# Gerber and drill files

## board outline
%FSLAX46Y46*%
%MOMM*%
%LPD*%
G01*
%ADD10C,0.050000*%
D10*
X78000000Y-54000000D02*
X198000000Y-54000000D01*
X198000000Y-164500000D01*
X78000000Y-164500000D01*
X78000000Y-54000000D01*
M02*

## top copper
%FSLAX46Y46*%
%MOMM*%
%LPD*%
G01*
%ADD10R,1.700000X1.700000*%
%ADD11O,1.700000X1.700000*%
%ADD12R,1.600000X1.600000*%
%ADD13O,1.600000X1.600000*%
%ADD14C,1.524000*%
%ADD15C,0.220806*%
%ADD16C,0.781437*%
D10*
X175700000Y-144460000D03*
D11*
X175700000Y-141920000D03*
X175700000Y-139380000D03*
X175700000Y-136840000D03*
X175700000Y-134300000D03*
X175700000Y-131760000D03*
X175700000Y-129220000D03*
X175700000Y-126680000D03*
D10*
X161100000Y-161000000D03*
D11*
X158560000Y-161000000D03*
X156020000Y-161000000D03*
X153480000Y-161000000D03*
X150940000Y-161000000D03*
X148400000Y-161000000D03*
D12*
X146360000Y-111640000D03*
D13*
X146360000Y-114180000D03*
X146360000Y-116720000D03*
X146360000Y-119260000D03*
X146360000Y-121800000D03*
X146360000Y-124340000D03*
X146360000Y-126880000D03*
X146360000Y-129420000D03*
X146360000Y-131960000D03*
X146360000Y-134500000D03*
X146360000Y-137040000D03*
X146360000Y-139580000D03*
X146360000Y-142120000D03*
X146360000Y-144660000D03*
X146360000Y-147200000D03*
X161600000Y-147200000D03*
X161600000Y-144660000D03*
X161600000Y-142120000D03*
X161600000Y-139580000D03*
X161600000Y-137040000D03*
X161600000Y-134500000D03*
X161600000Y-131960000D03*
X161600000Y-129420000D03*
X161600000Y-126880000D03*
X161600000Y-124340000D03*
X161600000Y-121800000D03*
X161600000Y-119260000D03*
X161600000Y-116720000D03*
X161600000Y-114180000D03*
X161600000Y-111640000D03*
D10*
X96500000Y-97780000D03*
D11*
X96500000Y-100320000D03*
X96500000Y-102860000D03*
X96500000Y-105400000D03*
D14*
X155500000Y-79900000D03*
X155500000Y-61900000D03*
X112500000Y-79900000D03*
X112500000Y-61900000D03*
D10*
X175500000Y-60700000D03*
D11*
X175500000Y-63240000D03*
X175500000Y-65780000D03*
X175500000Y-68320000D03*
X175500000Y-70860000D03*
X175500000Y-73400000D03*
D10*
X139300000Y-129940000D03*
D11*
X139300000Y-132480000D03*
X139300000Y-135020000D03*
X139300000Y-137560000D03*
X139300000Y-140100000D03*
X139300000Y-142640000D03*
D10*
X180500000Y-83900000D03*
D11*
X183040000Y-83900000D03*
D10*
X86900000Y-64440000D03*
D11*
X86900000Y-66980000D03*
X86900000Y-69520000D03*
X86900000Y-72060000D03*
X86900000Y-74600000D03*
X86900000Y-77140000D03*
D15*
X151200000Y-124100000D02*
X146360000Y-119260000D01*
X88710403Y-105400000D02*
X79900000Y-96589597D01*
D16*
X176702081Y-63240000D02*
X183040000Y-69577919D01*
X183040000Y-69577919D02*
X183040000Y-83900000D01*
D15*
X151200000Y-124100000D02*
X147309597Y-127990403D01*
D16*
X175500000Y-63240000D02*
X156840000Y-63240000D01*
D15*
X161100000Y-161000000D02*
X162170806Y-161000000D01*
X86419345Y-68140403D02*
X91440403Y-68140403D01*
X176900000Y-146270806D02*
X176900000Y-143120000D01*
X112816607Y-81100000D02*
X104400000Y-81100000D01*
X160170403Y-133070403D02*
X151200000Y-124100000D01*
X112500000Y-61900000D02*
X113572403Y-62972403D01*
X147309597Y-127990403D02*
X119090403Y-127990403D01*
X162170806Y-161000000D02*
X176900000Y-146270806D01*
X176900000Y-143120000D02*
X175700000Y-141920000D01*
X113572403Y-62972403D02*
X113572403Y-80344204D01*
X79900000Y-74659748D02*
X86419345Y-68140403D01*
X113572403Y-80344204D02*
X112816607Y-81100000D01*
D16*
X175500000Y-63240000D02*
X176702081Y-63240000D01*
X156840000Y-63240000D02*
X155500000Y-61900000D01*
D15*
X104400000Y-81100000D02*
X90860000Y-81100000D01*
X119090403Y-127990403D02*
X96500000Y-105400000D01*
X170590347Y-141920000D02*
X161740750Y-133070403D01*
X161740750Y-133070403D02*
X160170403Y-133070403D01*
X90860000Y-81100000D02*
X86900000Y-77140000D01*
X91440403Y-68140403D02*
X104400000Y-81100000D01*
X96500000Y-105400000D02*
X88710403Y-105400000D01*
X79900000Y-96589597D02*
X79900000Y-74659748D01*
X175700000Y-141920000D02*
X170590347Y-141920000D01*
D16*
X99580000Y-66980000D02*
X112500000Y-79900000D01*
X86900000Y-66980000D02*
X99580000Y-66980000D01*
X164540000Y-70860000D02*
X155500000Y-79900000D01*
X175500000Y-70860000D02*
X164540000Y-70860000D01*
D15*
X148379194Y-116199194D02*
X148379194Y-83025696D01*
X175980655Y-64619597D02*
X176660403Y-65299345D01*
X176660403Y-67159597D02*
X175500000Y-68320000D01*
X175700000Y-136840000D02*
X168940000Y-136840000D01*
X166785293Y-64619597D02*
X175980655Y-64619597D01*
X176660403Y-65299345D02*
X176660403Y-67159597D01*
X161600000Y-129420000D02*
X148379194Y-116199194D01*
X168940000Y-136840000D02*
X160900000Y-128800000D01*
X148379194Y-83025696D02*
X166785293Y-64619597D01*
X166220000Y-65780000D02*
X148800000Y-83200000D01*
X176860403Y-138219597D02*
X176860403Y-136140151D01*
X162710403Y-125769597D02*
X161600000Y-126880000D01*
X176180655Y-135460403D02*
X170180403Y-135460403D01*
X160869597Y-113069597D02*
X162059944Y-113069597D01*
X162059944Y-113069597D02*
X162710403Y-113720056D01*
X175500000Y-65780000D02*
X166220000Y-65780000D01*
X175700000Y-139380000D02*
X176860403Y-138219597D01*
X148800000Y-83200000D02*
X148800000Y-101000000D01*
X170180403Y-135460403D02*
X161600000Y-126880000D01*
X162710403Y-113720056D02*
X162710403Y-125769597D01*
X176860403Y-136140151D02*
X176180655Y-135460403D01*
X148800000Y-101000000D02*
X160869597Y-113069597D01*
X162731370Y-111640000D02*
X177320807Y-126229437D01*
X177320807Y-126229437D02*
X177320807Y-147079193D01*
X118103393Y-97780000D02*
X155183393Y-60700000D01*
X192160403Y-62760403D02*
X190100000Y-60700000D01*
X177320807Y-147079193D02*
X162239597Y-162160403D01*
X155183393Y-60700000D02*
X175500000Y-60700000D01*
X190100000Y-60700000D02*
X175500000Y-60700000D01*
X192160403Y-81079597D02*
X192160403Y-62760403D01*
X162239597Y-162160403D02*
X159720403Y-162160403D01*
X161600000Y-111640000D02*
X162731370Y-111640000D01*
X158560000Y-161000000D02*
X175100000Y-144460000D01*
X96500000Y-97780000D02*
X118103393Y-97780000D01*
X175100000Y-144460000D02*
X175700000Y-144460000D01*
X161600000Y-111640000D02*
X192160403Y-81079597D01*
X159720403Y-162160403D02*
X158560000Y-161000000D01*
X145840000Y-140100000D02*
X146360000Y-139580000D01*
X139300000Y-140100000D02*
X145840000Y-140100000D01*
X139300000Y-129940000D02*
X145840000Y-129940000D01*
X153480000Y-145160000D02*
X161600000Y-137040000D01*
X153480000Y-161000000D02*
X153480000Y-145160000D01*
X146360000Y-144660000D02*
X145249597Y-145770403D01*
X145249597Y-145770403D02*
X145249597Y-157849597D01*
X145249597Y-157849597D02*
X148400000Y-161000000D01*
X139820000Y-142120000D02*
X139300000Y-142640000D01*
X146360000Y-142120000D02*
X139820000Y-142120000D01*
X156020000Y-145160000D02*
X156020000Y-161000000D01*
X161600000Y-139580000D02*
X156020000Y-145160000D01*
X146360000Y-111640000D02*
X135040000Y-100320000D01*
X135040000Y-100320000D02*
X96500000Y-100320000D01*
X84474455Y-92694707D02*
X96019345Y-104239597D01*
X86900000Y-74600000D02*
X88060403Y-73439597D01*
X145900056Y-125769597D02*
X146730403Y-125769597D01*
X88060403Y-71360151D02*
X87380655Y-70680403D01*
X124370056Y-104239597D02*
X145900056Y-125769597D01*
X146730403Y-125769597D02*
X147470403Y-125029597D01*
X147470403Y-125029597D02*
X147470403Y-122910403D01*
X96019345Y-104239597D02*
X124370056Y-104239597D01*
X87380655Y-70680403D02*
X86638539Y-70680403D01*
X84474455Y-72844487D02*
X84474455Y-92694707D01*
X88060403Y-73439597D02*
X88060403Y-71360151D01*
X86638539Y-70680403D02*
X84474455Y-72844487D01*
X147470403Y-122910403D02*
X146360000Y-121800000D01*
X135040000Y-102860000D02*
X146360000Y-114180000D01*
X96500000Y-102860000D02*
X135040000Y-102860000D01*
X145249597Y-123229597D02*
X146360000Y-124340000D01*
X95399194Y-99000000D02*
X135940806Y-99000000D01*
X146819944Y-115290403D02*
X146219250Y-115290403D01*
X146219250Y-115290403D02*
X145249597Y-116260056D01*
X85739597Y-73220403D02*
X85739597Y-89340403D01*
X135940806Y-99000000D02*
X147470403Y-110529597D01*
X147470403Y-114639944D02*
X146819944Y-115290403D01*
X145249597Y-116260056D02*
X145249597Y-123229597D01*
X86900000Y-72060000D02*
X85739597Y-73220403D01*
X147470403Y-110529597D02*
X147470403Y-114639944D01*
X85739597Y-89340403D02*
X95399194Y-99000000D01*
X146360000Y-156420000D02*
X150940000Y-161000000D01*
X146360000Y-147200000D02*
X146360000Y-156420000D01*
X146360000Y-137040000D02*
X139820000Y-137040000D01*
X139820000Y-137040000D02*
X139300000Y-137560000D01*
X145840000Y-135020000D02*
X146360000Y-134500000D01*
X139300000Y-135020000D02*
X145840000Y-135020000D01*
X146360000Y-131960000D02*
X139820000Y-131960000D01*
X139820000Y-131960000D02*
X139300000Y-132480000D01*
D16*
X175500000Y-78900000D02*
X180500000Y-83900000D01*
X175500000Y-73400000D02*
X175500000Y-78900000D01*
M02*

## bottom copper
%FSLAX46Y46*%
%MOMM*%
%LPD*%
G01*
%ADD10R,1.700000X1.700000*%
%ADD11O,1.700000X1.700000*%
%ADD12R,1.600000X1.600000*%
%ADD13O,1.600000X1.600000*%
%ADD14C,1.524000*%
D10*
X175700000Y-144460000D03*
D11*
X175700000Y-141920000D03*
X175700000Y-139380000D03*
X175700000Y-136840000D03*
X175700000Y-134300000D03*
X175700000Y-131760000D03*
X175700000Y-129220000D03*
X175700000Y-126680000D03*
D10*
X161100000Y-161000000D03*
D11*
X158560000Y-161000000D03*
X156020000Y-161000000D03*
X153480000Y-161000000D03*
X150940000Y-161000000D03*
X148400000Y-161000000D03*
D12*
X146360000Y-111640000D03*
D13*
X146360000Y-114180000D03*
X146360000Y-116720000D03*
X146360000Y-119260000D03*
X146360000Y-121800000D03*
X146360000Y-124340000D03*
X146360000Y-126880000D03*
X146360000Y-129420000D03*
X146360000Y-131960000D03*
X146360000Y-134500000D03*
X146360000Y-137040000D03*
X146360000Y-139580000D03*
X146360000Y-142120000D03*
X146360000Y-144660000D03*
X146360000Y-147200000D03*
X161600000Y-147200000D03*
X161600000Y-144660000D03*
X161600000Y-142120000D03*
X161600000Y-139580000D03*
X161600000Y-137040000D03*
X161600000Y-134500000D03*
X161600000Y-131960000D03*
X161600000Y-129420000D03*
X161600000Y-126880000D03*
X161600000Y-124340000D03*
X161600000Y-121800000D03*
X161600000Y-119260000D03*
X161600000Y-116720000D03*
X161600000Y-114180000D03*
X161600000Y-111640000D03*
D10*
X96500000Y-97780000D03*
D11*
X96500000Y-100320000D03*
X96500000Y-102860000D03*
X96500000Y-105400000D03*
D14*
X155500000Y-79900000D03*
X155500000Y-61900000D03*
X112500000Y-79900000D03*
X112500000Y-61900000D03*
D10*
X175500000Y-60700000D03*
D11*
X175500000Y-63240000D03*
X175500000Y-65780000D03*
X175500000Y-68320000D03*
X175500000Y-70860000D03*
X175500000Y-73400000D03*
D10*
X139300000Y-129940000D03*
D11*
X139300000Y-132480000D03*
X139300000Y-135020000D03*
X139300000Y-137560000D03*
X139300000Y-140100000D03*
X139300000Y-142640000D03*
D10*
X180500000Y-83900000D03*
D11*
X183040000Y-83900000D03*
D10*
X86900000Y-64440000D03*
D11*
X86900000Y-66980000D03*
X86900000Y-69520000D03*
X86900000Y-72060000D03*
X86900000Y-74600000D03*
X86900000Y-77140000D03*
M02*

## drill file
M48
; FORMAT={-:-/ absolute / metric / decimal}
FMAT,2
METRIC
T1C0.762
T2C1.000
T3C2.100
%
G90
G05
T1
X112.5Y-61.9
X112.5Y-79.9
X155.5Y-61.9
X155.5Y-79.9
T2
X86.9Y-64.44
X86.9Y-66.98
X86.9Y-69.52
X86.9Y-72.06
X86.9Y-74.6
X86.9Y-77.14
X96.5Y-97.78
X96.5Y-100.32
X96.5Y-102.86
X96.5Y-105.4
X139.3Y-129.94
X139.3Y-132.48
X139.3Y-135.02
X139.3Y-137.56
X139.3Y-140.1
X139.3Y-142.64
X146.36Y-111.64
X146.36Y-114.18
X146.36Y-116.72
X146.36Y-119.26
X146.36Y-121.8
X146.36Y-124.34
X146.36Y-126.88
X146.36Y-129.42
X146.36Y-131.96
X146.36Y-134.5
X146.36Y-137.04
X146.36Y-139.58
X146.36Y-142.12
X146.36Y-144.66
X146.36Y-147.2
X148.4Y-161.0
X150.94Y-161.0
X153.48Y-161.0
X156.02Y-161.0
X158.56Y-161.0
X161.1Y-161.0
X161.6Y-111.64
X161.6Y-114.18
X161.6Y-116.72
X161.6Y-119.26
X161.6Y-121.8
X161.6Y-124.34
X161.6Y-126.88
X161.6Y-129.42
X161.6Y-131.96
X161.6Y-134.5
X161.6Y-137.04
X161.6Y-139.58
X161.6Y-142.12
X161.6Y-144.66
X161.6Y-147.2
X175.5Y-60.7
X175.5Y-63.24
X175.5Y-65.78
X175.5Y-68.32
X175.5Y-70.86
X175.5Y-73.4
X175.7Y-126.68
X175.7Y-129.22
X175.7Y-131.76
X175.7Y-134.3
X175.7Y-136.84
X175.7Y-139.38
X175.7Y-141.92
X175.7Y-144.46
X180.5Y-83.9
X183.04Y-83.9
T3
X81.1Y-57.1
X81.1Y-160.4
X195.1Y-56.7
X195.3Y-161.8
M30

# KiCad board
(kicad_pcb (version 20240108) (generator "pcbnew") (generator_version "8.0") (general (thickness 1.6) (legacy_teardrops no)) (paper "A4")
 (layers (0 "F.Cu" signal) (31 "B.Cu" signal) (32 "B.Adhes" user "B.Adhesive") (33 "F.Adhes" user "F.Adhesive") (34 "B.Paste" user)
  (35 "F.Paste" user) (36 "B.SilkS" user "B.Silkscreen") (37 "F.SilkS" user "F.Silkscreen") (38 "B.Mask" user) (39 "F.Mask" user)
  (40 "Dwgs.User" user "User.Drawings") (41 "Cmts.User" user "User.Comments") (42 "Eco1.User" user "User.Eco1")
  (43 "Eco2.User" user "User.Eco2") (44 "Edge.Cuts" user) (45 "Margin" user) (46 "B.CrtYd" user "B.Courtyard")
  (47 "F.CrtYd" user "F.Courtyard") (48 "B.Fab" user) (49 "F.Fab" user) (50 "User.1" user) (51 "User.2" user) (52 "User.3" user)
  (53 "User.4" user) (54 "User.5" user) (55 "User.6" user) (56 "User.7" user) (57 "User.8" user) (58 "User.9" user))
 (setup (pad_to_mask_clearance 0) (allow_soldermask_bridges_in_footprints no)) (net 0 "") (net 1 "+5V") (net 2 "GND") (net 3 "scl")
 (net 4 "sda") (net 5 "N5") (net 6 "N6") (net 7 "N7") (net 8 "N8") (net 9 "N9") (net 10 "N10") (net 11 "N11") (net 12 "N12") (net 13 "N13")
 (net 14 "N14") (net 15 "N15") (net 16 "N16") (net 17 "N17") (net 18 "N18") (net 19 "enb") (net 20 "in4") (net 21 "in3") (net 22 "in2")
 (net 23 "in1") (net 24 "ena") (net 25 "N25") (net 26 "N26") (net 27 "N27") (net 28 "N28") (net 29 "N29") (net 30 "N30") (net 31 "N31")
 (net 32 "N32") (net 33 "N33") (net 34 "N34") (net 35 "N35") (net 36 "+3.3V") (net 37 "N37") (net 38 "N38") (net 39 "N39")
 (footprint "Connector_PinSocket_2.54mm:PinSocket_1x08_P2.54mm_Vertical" (layer "F.Cu") (at 175.7 144.46 180)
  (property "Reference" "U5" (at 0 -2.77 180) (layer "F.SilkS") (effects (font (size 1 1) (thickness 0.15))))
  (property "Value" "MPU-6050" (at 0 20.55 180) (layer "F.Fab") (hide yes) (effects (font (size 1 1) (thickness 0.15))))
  (pad "1" thru_hole rect (at 0 0 180) (size 1.7 1.7) (drill 1) (layers "*.Cu" "*.Mask") (remove_unused_layers no) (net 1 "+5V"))
  (pad "2" thru_hole oval (at 0 2.54 180) (size 1.7 1.7) (drill 1) (layers "*.Cu" "*.Mask") (remove_unused_layers no) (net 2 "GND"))
  (pad "3" thru_hole oval (at 0 5.08 180) (size 1.7 1.7) (drill 1) (layers "*.Cu" "*.Mask") (remove_unused_layers no) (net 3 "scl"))
  (pad "4" thru_hole oval (at 0 7.62 180) (size 1.7 1.7) (drill 1) (layers "*.Cu" "*.Mask") (remove_unused_layers no) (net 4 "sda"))
  (pad "5" thru_hole oval (at 0 10.16 180) (size 1.7 1.7) (drill 1) (layers "*.Cu" "*.Mask") (remove_unused_layers no) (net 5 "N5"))
  (pad "6" thru_hole oval (at 0 12.7 180) (size 1.7 1.7) (drill 1) (layers "*.Cu" "*.Mask") (remove_unused_layers no) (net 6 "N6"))
  (pad "7" thru_hole oval (at 0 15.24 180) (size 1.7 1.7) (drill 1) (layers "*.Cu" "*.Mask") (remove_unused_layers no) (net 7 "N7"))
  (pad "8" thru_hole oval (at 0 17.78 180) (size 1.7 1.7) (drill 1) (layers "*.Cu" "*.Mask") (remove_unused_layers no) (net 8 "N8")))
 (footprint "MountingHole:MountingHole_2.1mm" (layer "F.Cu") (at 81.1 160.4)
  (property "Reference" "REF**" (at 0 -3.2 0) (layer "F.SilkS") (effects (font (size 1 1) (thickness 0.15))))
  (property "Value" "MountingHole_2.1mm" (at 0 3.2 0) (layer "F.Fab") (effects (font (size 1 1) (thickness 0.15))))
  (pad "" np_thru_hole circle (at 0 0) (size 2.1 2.1) (drill 2.1) (layers "*.Cu" "*.Mask")))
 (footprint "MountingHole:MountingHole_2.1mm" (layer "F.Cu") (at 81.1 57.1)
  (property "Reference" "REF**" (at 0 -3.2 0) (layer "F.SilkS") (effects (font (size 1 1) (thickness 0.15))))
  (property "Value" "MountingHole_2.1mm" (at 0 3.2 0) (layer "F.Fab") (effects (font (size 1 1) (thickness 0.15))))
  (pad "" np_thru_hole circle (at 0 0) (size 2.1 2.1) (drill 2.1) (layers "*.Cu" "*.Mask")))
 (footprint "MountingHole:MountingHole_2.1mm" (layer "F.Cu") (at 195.1 56.7)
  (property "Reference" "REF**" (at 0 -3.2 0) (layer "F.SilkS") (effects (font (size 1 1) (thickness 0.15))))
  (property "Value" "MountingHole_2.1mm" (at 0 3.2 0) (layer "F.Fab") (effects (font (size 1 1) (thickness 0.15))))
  (pad "" np_thru_hole circle (at 0 0) (size 2.1 2.1) (drill 2.1) (layers "*.Cu" "*.Mask")))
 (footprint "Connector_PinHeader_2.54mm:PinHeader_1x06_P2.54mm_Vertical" (layer "F.Cu") (at 161.1 161 -90)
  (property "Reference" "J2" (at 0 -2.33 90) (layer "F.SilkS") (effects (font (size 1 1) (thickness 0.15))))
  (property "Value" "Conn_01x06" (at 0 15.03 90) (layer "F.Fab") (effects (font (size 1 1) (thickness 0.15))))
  (pad "1" thru_hole rect (at 0 0 270) (size 1.7 1.7) (drill 1) (layers "*.Cu" "*.Mask") (remove_unused_layers no) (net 2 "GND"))
  (pad "2" thru_hole oval (at 0 2.54 270) (size 1.7 1.7) (drill 1) (layers "*.Cu" "*.Mask") (remove_unused_layers no) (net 1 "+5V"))
  (pad "3" thru_hole oval (at 0 5.08 270) (size 1.7 1.7) (drill 1) (layers "*.Cu" "*.Mask") (remove_unused_layers no) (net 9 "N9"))
  (pad "4" thru_hole oval (at 0 7.62 270) (size 1.7 1.7) (drill 1) (layers "*.Cu" "*.Mask") (remove_unused_layers no) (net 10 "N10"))
  (pad "5" thru_hole oval (at 0 10.16 270) (size 1.7 1.7) (drill 1) (layers "*.Cu" "*.Mask") (remove_unused_layers no) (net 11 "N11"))
  (pad "6" thru_hole oval (at 0 12.7 270) (size 1.7 1.7) (drill 1) (layers "*.Cu" "*.Mask") (remove_unused_layers no) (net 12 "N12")))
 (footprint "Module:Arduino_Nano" (layer "F.Cu") (at 146.36 111.64)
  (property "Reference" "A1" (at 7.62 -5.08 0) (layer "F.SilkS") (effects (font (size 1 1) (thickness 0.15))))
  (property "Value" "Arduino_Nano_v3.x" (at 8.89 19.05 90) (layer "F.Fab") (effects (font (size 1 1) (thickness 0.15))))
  (pad "1" thru_hole rect (at 0 0) (size 1.6 1.6) (drill 1) (layers "*.Cu" "*.Mask") (remove_unused_layers no) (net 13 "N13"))
  (pad "2" thru_hole oval (at 0 2.54) (size 1.6 1.6) (drill 1) (layers "*.Cu" "*.Mask") (remove_unused_layers no) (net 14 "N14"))
  (pad "3" thru_hole oval (at 0 5.08) (size 1.6 1.6) (drill 1) (layers "*.Cu" "*.Mask") (remove_unused_layers no) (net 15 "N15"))
  (pad "4" thru_hole oval (at 0 7.62) (size 1.6 1.6) (drill 1) (layers "*.Cu" "*.Mask") (remove_unused_layers no) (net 2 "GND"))
  (pad "5" thru_hole oval (at 0 10.16) (size 1.6 1.6) (drill 1) (layers "*.Cu" "*.Mask") (remove_unused_layers no) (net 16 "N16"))
  (pad "6" thru_hole oval (at 0 12.7) (size 1.6 1.6) (drill 1) (layers "*.Cu" "*.Mask") (remove_unused_layers no) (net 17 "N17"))
  (pad "7" thru_hole oval (at 0 15.24) (size 1.6 1.6) (drill 1) (layers "*.Cu" "*.Mask") (remove_unused_layers no) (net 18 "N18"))
  (pad "8" thru_hole oval (at 0 17.78) (size 1.6 1.6) (drill 1) (layers "*.Cu" "*.Mask") (remove_unused_layers no) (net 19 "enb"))
  (pad "9" thru_hole oval (at 0 20.32) (size 1.6 1.6) (drill 1) (layers "*.Cu" "*.Mask") (remove_unused_layers no) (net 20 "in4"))
  (pad "10" thru_hole oval (at 0 22.86) (size 1.6 1.6) (drill 1) (layers "*.Cu" "*.Mask") (remove_unused_layers no) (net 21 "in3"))
  (pad "11" thru_hole oval (at 0 25.4) (size 1.6 1.6) (drill 1) (layers "*.Cu" "*.Mask") (remove_unused_layers no) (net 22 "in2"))
  (pad "12" thru_hole oval (at 0 27.94) (size 1.6 1.6) (drill 1) (layers "*.Cu" "*.Mask") (remove_unused_layers no) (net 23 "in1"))
  (pad "13" thru_hole oval (at 0 30.48) (size 1.6 1.6) (drill 1) (layers "*.Cu" "*.Mask") (remove_unused_layers no) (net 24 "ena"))
  (pad "14" thru_hole oval (at 0 33.02) (size 1.6 1.6) (drill 1) (layers "*.Cu" "*.Mask") (remove_unused_layers no) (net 12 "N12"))
  (pad "15" thru_hole oval (at 0 35.56) (size 1.6 1.6) (drill 1) (layers "*.Cu" "*.Mask") (remove_unused_layers no) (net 11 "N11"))
  (pad "16" thru_hole oval (at 15.24 35.56) (size 1.6 1.6) (drill 1) (layers "*.Cu" "*.Mask") (remove_unused_layers no) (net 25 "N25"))
  (pad "17" thru_hole oval (at 15.24 33.02) (size 1.6 1.6) (drill 1) (layers "*.Cu" "*.Mask") (remove_unused_layers no) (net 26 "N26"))
  (pad "18" thru_hole oval (at 15.24 30.48) (size 1.6 1.6) (drill 1) (layers "*.Cu" "*.Mask") (remove_unused_layers no) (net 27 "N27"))
  (pad "19" thru_hole oval (at 15.24 27.94) (size 1.6 1.6) (drill 1) (layers "*.Cu" "*.Mask") (remove_unused_layers no) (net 9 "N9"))
  (pad "20" thru_hole oval (at 15.24 25.4) (size 1.6 1.6) (drill 1) (layers "*.Cu" "*.Mask") (remove_unused_layers no) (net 10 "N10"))
  (pad "21" thru_hole oval (at 15.24 22.86) (size 1.6 1.6) (drill 1) (layers "*.Cu" "*.Mask") (remove_unused_layers no) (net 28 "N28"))
  (pad "22" thru_hole oval (at 15.24 20.32) (size 1.6 1.6) (drill 1) (layers "*.Cu" "*.Mask") (remove_unused_layers no) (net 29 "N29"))
  (pad "23" thru_hole oval (at 15.24 17.78) (size 1.6 1.6) (drill 1) (layers "*.Cu" "*.Mask") (remove_unused_layers no) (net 4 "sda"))
  (pad "24" thru_hole oval (at 15.24 15.24) (size 1.6 1.6) (drill 1) (layers "*.Cu" "*.Mask") (remove_unused_layers no) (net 3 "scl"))
  (pad "25" thru_hole oval (at 15.24 12.7) (size 1.6 1.6) (drill 1) (layers "*.Cu" "*.Mask") (remove_unused_layers no) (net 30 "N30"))
  (pad "26" thru_hole oval (at 15.24 10.16) (size 1.6 1.6) (drill 1) (layers "*.Cu" "*.Mask") (remove_unused_layers no) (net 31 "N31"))
  (pad "27" thru_hole oval (at 15.24 7.62) (size 1.6 1.6) (drill 1) (layers "*.Cu" "*.Mask") (remove_unused_layers no) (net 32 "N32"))
  (pad "28" thru_hole oval (at 15.24 5.08) (size 1.6 1.6) (drill 1) (layers "*.Cu" "*.Mask") (remove_unused_layers no) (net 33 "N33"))
  (pad "29" thru_hole oval (at 15.24 2.54) (size 1.6 1.6) (drill 1) (layers "*.Cu" "*.Mask") (remove_unused_layers no) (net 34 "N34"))
  (pad "30" thru_hole oval (at 15.24 0) (size 1.6 1.6) (drill 1) (layers "*.Cu" "*.Mask") (remove_unused_layers no) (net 1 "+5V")))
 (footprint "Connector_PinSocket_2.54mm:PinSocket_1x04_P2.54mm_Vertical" (layer "F.Cu") (at 96.5 97.78)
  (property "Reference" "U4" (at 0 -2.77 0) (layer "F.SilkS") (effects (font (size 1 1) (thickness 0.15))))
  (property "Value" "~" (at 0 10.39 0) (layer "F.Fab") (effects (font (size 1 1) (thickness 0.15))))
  (pad "1" thru_hole rect (at 0 0) (size 1.7 1.7) (drill 1) (layers "*.Cu" "*.Mask") (remove_unused_layers no) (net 1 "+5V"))
  (pad "2" thru_hole oval (at 0 2.54) (size 1.7 1.7) (drill 1) (layers "*.Cu" "*.Mask") (remove_unused_layers no) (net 13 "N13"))
  (pad "3" thru_hole oval (at 0 5.08) (size 1.7 1.7) (drill 1) (layers "*.Cu" "*.Mask") (remove_unused_layers no) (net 14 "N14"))
  (pad "4" thru_hole oval (at 0 7.62) (size 1.7 1.7) (drill 1) (layers "*.Cu" "*.Mask") (remove_unused_layers no) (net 2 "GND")))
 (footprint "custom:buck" (layer "F.Cu") (at 134 70.4 180)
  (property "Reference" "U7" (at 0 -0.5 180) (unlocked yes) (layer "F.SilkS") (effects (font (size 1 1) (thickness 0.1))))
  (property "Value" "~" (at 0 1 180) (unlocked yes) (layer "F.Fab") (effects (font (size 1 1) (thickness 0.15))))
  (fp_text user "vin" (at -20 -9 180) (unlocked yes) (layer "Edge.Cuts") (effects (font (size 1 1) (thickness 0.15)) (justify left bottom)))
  (pad "1" thru_hole circle (at -21.5 -9.5 180) (size 1.524 1.524) (drill 0.762) (layers "*.Cu" "*.Mask") (remove_unused_layers no)
   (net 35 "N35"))
  (pad "2" thru_hole circle (at -21.5 8.5 180) (size 1.524 1.524) (drill 0.762) (layers "*.Cu" "*.Mask") (remove_unused_layers no)
   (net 2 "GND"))
  (pad "3" thru_hole circle (at 21.5 -9.5 180) (size 1.524 1.524) (drill 0.762) (layers "*.Cu" "*.Mask") (remove_unused_layers no)
   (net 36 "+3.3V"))
  (pad "4" thru_hole circle (at 21.5 8.5 180) (size 1.524 1.524) (drill 0.762) (layers "*.Cu" "*.Mask") (remove_unused_layers no)
   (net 2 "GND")))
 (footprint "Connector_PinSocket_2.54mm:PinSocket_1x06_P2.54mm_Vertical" (layer "F.Cu") (at 175.5 60.7)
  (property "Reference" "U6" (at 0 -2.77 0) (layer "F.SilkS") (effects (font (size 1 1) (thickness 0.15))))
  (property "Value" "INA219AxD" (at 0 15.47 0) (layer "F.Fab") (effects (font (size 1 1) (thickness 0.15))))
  (pad "1" thru_hole rect (at 0 0) (size 1.7 1.7) (drill 1) (layers "*.Cu" "*.Mask") (remove_unused_layers no) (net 1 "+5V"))
  (pad "2" thru_hole oval (at 0 2.54) (size 1.7 1.7) (drill 1) (layers "*.Cu" "*.Mask") (remove_unused_layers no) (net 2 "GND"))
  (pad "3" thru_hole oval (at 0 5.08) (size 1.7 1.7) (drill 1) (layers "*.Cu" "*.Mask") (remove_unused_layers no) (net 3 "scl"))
  (pad "4" thru_hole oval (at 0 7.62) (size 1.7 1.7) (drill 1) (layers "*.Cu" "*.Mask") (remove_unused_layers no) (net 4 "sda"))
  (pad "5" thru_hole oval (at 0 10.16) (size 1.7 1.7) (drill 1) (layers "*.Cu" "*.Mask") (remove_unused_layers no) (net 35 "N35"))
  (pad "6" thru_hole oval (at 0 12.7) (size 1.7 1.7) (drill 1) (layers "*.Cu" "*.Mask") (remove_unused_layers no) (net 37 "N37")))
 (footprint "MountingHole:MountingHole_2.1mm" (layer "F.Cu") (at 195.3 161.8)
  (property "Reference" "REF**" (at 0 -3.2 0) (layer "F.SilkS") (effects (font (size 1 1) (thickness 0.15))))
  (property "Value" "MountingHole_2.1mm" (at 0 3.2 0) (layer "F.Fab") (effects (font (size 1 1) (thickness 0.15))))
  (pad "" np_thru_hole circle (at 0 0) (size 2.1 2.1) (drill 2.1) (layers "*.Cu" "*.Mask")))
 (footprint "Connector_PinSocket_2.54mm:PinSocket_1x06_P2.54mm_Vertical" (layer "F.Cu") (at 139.3 129.94)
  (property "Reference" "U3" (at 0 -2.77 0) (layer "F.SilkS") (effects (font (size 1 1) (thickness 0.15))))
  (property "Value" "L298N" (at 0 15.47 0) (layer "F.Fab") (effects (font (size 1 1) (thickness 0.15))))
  (pad "1" thru_hole rect (at 0 0) (size 1.7 1.7) (drill 1) (layers "*.Cu" "*.Mask") (remove_unused_layers no) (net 19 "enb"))
  (pad "2" thru_hole oval (at 0 2.54) (size 1.7 1.7) (drill 1) (layers "*.Cu" "*.Mask") (remove_unused_layers no) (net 20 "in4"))
  (pad "3" thru_hole oval (at 0 5.08) (size 1.7 1.7) (drill 1) (layers "*.Cu" "*.Mask") (remove_unused_layers no) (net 21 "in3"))
  (pad "4" thru_hole oval (at 0 7.62) (size 1.7 1.7) (drill 1) (layers "*.Cu" "*.Mask") (remove_unused_layers no) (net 22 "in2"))
  (pad "5" thru_hole oval (at 0 10.16) (size 1.7 1.7) (drill 1) (layers "*.Cu" "*.Mask") (remove_unused_layers no) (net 23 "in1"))
  (pad "6" thru_hole oval (at 0 12.7) (size 1.7 1.7) (drill 1) (layers "*.Cu" "*.Mask") (remove_unused_layers no) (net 24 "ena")))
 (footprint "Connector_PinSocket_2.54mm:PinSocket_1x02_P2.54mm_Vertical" (layer "F.Cu") (at 180.5 83.9 90)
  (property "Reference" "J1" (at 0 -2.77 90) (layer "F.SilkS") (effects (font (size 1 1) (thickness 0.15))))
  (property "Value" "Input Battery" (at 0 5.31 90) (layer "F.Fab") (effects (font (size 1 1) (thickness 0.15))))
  (pad "1" thru_hole rect (at 0 0 90) (size 1.7 1.7) (drill 1) (layers "*.Cu" "*.Mask") (remove_unused_layers no) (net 37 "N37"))
  (pad "2" thru_hole oval (at 0 2.54 90) (size 1.7 1.7) (drill 1) (layers "*.Cu" "*.Mask") (remove_unused_layers no) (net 2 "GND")))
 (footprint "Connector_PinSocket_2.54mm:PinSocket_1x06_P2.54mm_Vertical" (layer "F.Cu") (at 86.9 64.44)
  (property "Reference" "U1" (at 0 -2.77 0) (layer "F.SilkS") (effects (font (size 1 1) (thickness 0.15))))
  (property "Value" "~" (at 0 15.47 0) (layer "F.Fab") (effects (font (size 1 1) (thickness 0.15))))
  (pad "1" thru_hole rect (at 0 0) (size 1.7 1.7) (drill 1) (layers "*.Cu" "*.Mask") (remove_unused_layers no) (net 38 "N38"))
  (pad "2" thru_hole oval (at 0 2.54) (size 1.7 1.7) (drill 1) (layers "*.Cu" "*.Mask") (remove_unused_layers no) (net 36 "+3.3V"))
  (pad "3" thru_hole oval (at 0 5.08) (size 1.7 1.7) (drill 1) (layers "*.Cu" "*.Mask") (remove_unused_layers no) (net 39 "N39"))
  (pad "4" thru_hole oval (at 0 7.62) (size 1.7 1.7) (drill 1) (layers "*.Cu" "*.Mask") (remove_unused_layers no) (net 17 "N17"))
  (pad "5" thru_hole oval (at 0 10.16) (size 1.7 1.7) (drill 1) (layers "*.Cu" "*.Mask") (remove_unused_layers no) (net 16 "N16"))
  (pad "6" thru_hole oval (at 0 12.7) (size 1.7 1.7) (drill 1) (layers "*.Cu" "*.Mask") (remove_unused_layers no) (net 2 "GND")))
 (gr_rect (start 78 54) (end 198 164.5) (stroke (width 0.05) (type default)) (fill none) (layer "Edge.Cuts"))
 (segment (start 151.2 124.1) (end 146.36 119.26) (width 0.220806) (layer "F.Cu") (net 2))
 (segment (start 88.710403 105.4) (end 79.9 96.589597) (width 0.220806) (layer "F.Cu") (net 2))
 (segment (start 176.702081 63.24) (end 183.04 69.577919) (width 0.781437) (layer "F.Cu") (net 2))
 (segment (start 183.04 69.577919) (end 183.04 83.9) (width 0.781437) (layer "F.Cu") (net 2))
 (segment (start 151.2 124.1) (end 147.309597 127.990403) (width 0.220806) (layer "F.Cu") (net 2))
 (segment (start 175.5 63.24) (end 156.84 63.24) (width 0.781437) (layer "F.Cu") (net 2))
 (segment (start 161.1 161) (end 162.170806 161) (width 0.220806) (layer "F.Cu") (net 2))
 (segment (start 86.419345 68.140403) (end 91.440403 68.140403) (width 0.220806) (layer "F.Cu") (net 2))
 (segment (start 176.9 146.270806) (end 176.9 143.12) (width 0.220806) (layer "F.Cu") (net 2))
 (segment (start 112.816607 81.1) (end 104.4 81.1) (width 0.220806) (layer "F.Cu") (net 2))
 (segment (start 160.170403 133.070403) (end 151.2 124.1) (width 0.220806) (layer "F.Cu") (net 2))
 (segment (start 112.5 61.9) (end 113.572403 62.972403) (width 0.220806) (layer "F.Cu") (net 2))
 (segment (start 147.309597 127.990403) (end 119.090403 127.990403) (width 0.220806) (layer "F.Cu") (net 2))
 (segment (start 162.170806 161) (end 176.9 146.270806) (width 0.220806) (layer "F.Cu") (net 2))
 (segment (start 176.9 143.12) (end 175.7 141.92) (width 0.220806) (layer "F.Cu") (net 2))
 (segment (start 113.572403 62.972403) (end 113.572403 80.344204) (width 0.220806) (layer "F.Cu") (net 2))
 (segment (start 79.9 74.659748) (end 86.419345 68.140403) (width 0.220806) (layer "F.Cu") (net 2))
 (segment (start 113.572403 80.344204) (end 112.816607 81.1) (width 0.220806) (layer "F.Cu") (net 2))
 (segment (start 175.5 63.24) (end 176.702081 63.24) (width 0.781437) (layer "F.Cu") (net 2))
 (segment (start 156.84 63.24) (end 155.5 61.9) (width 0.781437) (layer "F.Cu") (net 2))
 (segment (start 104.4 81.1) (end 90.86 81.1) (width 0.220806) (layer "F.Cu") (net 2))
 (segment (start 119.090403 127.990403) (end 96.5 105.4) (width 0.220806) (layer "F.Cu") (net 2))
 (segment (start 170.590347 141.92) (end 161.74075 133.070403) (width 0.220806) (layer "F.Cu") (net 2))
 (segment (start 161.74075 133.070403) (end 160.170403 133.070403) (width 0.220806) (layer "F.Cu") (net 2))
 (segment (start 90.86 81.1) (end 86.9 77.14) (width 0.220806) (layer "F.Cu") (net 2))
 (segment (start 91.440403 68.140403) (end 104.4 81.1) (width 0.220806) (layer "F.Cu") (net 2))
 (segment (start 96.5 105.4) (end 88.710403 105.4) (width 0.220806) (layer "F.Cu") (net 2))
 (segment (start 79.9 96.589597) (end 79.9 74.659748) (width 0.220806) (layer "F.Cu") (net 2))
 (segment (start 175.7 141.92) (end 170.590347 141.92) (width 0.220806) (layer "F.Cu") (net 2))
 (segment (start 99.58 66.98) (end 112.5 79.9) (width 0.781437) (layer "F.Cu") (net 36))
 (segment (start 86.9 66.98) (end 99.58 66.98) (width 0.781437) (layer "F.Cu") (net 36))
 (segment (start 164.54 70.86) (end 155.5 79.9) (width 0.781437) (layer "F.Cu") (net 35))
 (segment (start 175.5 70.86) (end 164.54 70.86) (width 0.781437) (layer "F.Cu") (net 35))
 (segment (start 148.379194 116.199194) (end 148.379194 83.025696) (width 0.220806) (layer "F.Cu") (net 4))
 (segment (start 175.980655 64.619597) (end 176.660403 65.299345) (width 0.220806) (layer "F.Cu") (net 4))
 (segment (start 176.660403 67.159597) (end 175.5 68.32) (width 0.220806) (layer "F.Cu") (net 4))
 (segment (start 175.7 136.84) (end 168.94 136.84) (width 0.220806) (layer "F.Cu") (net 4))
 (segment (start 166.785293 64.619597) (end 175.980655 64.619597) (width 0.220806) (layer "F.Cu") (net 4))
 (segment (start 176.660403 65.299345) (end 176.660403 67.159597) (width 0.220806) (layer "F.Cu") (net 4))
 (segment (start 161.6 129.42) (end 148.379194 116.199194) (width 0.220806) (layer "F.Cu") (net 4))
 (segment (start 168.94 136.84) (end 160.9 128.8) (width 0.220806) (layer "F.Cu") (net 4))
 (segment (start 148.379194 83.025696) (end 166.785293 64.619597) (width 0.220806) (layer "F.Cu") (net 4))
 (segment (start 166.22 65.78) (end 148.8 83.2) (width 0.220806) (layer "F.Cu") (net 3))
 (segment (start 176.860403 138.219597) (end 176.860403 136.140151) (width 0.220806) (layer "F.Cu") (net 3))
 (segment (start 162.710403 125.769597) (end 161.6 126.88) (width 0.220806) (layer "F.Cu") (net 3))
 (segment (start 176.180655 135.460403) (end 170.180403 135.460403) (width 0.220806) (layer "F.Cu") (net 3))
 (segment (start 160.869597 113.069597) (end 162.059944 113.069597) (width 0.220806) (layer "F.Cu") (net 3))
 (segment (start 162.059944 113.069597) (end 162.710403 113.720056) (width 0.220806) (layer "F.Cu") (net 3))
 (segment (start 175.5 65.78) (end 166.22 65.78) (width 0.220806) (layer "F.Cu") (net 3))
 (segment (start 175.7 139.38) (end 176.860403 138.219597) (width 0.220806) (layer "F.Cu") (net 3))
 (segment (start 148.8 83.2) (end 148.8 101) (width 0.220806) (layer "F.Cu") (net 3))
 (segment (start 170.180403 135.460403) (end 161.6 126.88) (width 0.220806) (layer "F.Cu") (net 3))
 (segment (start 162.710403 113.720056) (end 162.710403 125.769597) (width 0.220806) (layer "F.Cu") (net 3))
 (segment (start 176.860403 136.140151) (end 176.180655 135.460403) (width 0.220806) (layer "F.Cu") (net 3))
 (segment (start 148.8 101) (end 160.869597 113.069597) (width 0.220806) (layer "F.Cu") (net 3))
 (segment (start 162.73137 111.64) (end 177.320807 126.229437) (width 0.220806) (layer "F.Cu") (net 1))
 (segment (start 177.320807 126.229437) (end 177.320807 147.079193) (width 0.220806) (layer "F.Cu") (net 1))
 (segment (start 118.103393 97.78) (end 155.183393 60.7) (width 0.220806) (layer "F.Cu") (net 1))
 (segment (start 192.160403 62.760403) (end 190.1 60.7) (width 0.220806) (layer "F.Cu") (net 1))
 (segment (start 177.320807 147.079193) (end 162.239597 162.160403) (width 0.220806) (layer "F.Cu") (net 1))
 (segment (start 155.183393 60.7) (end 175.5 60.7) (width 0.220806) (layer "F.Cu") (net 1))
 (segment (start 190.1 60.7) (end 175.5 60.7) (width 0.220806) (layer "F.Cu") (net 1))
 (segment (start 192.160403 81.079597) (end 192.160403 62.760403) (width 0.220806) (layer "F.Cu") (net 1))
 (segment (start 162.239597 162.160403) (end 159.720403 162.160403) (width 0.220806) (layer "F.Cu") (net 1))
 (segment (start 161.6 111.64) (end 162.73137 111.64) (width 0.220806) (layer "F.Cu") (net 1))
 (segment (start 158.56 161) (end 175.1 144.46) (width 0.220806) (layer "F.Cu") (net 1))
 (segment (start 96.5 97.78) (end 118.103393 97.78) (width 0.220806) (layer "F.Cu") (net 1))
 (segment (start 175.1 144.46) (end 175.7 144.46) (width 0.220806) (layer "F.Cu") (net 1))
 (segment (start 161.6 111.64) (end 192.160403 81.079597) (width 0.220806) (layer "F.Cu") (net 1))
 (segment (start 159.720403 162.160403) (end 158.56 161) (width 0.220806) (layer "F.Cu") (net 1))
 (segment (start 145.84 140.1) (end 146.36 139.58) (width 0.220806) (layer "F.Cu") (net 23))
 (segment (start 139.3 140.1) (end 145.84 140.1) (width 0.220806) (layer "F.Cu") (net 23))
 (segment (start 139.3 129.94) (end 145.84 129.94) (width 0.220806) (layer "F.Cu") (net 19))
 (segment (start 153.48 145.16) (end 161.6 137.04) (width 0.220806) (layer "F.Cu") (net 10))
 (segment (start 153.48 161) (end 153.48 145.16) (width 0.220806) (layer "F.Cu") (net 10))
 (segment (start 146.36 144.66) (end 145.249597 145.770403) (width 0.220806) (layer "F.Cu") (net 12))
 (segment (start 145.249597 145.770403) (end 145.249597 157.849597) (width 0.220806) (layer "F.Cu") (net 12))
 (segment (start 145.249597 157.849597) (end 148.4 161) (width 0.220806) (layer "F.Cu") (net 12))
 (segment (start 139.82 142.12) (end 139.3 142.64) (width 0.220806) (layer "F.Cu") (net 24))
 (segment (start 146.36 142.12) (end 139.82 142.12) (width 0.220806) (layer "F.Cu") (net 24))
 (segment (start 156.02 145.16) (end 156.02 161) (width 0.220806) (layer "F.Cu") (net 9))
 (segment (start 161.6 139.58) (end 156.02 145.16) (width 0.220806) (layer "F.Cu") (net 9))
 (segment (start 146.36 111.64) (end 135.04 100.32) (width 0.220806) (layer "F.Cu") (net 13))
 (segment (start 135.04 100.32) (end 96.5 100.32) (width 0.220806) (layer "F.Cu") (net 13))
 (segment (start 84.474455 92.694707) (end 96.019345 104.239597) (width 0.220806) (layer "F.Cu") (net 16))
 (segment (start 86.9 74.6) (end 88.060403 73.439597) (width 0.220806) (layer "F.Cu") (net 16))
 (segment (start 145.900056 125.769597) (end 146.730403 125.769597) (width 0.220806) (layer "F.Cu") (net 16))
 (segment (start 88.060403 71.360151) (end 87.380655 70.680403) (width 0.220806) (layer "F.Cu") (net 16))
 (segment (start 124.370056 104.239597) (end 145.900056 125.769597) (width 0.220806) (layer "F.Cu") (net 16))
 (segment (start 146.730403 125.769597) (end 147.470403 125.029597) (width 0.220806) (layer "F.Cu") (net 16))
 (segment (start 147.470403 125.029597) (end 147.470403 122.910403) (width 0.220806) (layer "F.Cu") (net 16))
 (segment (start 96.019345 104.239597) (end 124.370056 104.239597) (width 0.220806) (layer "F.Cu") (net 16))
 (segment (start 87.380655 70.680403) (end 86.638539 70.680403) (width 0.220806) (layer "F.Cu") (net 16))
 (segment (start 84.474455 72.844487) (end 84.474455 92.694707) (width 0.220806) (layer "F.Cu") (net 16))
 (segment (start 88.060403 73.439597) (end 88.060403 71.360151) (width 0.220806) (layer "F.Cu") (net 16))
 (segment (start 86.638539 70.680403) (end 84.474455 72.844487) (width 0.220806) (layer "F.Cu") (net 16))
 (segment (start 147.470403 122.910403) (end 146.36 121.8) (width 0.220806) (layer "F.Cu") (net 16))
 (segment (start 135.04 102.86) (end 146.36 114.18) (width 0.220806) (layer "F.Cu") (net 14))
 (segment (start 96.5 102.86) (end 135.04 102.86) (width 0.220806) (layer "F.Cu") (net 14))
 (segment (start 145.249597 123.229597) (end 146.36 124.34) (width 0.220806) (layer "F.Cu") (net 17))
 (segment (start 95.399194 99) (end 135.940806 99) (width 0.220806) (layer "F.Cu") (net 17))
 (segment (start 146.819944 115.290403) (end 146.21925 115.290403) (width 0.220806) (layer "F.Cu") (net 17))
 (segment (start 146.21925 115.290403) (end 145.249597 116.260056) (width 0.220806) (layer "F.Cu") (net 17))
 (segment (start 85.739597 73.220403) (end 85.739597 89.340403) (width 0.220806) (layer "F.Cu") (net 17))
 (segment (start 135.940806 99) (end 147.470403 110.529597) (width 0.220806) (layer "F.Cu") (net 17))
 (segment (start 147.470403 114.639944) (end 146.819944 115.290403) (width 0.220806) (layer "F.Cu") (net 17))
 (segment (start 145.249597 116.260056) (end 145.249597 123.229597) (width 0.220806) (layer "F.Cu") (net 17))
 (segment (start 86.9 72.06) (end 85.739597 73.220403) (width 0.220806) (layer "F.Cu") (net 17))
 (segment (start 147.470403 110.529597) (end 147.470403 114.639944) (width 0.220806) (layer "F.Cu") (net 17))
 (segment (start 85.739597 89.340403) (end 95.399194 99) (width 0.220806) (layer "F.Cu") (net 17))
 (segment (start 146.36 156.42) (end 150.94 161) (width 0.220806) (layer "F.Cu") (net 11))
 (segment (start 146.36 147.2) (end 146.36 156.42) (width 0.220806) (layer "F.Cu") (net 11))
 (segment (start 146.36 137.04) (end 139.82 137.04) (width 0.220806) (layer "F.Cu") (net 22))
 (segment (start 139.82 137.04) (end 139.3 137.56) (width 0.220806) (layer "F.Cu") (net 22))
 (segment (start 145.84 135.02) (end 146.36 134.5) (width 0.220806) (layer "F.Cu") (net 21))
 (segment (start 139.3 135.02) (end 145.84 135.02) (width 0.220806) (layer "F.Cu") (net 21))
 (segment (start 146.36 131.96) (end 139.82 131.96) (width 0.220806) (layer "F.Cu") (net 20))
 (segment (start 139.82 131.96) (end 139.3 132.48) (width 0.220806) (layer "F.Cu") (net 20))
 (segment (start 175.5 78.9) (end 180.5 83.9) (width 0.781437) (layer "F.Cu") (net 37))
 (segment (start 175.5 73.4) (end 175.5 78.9) (width 0.781437) (layer "F.Cu") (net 37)))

